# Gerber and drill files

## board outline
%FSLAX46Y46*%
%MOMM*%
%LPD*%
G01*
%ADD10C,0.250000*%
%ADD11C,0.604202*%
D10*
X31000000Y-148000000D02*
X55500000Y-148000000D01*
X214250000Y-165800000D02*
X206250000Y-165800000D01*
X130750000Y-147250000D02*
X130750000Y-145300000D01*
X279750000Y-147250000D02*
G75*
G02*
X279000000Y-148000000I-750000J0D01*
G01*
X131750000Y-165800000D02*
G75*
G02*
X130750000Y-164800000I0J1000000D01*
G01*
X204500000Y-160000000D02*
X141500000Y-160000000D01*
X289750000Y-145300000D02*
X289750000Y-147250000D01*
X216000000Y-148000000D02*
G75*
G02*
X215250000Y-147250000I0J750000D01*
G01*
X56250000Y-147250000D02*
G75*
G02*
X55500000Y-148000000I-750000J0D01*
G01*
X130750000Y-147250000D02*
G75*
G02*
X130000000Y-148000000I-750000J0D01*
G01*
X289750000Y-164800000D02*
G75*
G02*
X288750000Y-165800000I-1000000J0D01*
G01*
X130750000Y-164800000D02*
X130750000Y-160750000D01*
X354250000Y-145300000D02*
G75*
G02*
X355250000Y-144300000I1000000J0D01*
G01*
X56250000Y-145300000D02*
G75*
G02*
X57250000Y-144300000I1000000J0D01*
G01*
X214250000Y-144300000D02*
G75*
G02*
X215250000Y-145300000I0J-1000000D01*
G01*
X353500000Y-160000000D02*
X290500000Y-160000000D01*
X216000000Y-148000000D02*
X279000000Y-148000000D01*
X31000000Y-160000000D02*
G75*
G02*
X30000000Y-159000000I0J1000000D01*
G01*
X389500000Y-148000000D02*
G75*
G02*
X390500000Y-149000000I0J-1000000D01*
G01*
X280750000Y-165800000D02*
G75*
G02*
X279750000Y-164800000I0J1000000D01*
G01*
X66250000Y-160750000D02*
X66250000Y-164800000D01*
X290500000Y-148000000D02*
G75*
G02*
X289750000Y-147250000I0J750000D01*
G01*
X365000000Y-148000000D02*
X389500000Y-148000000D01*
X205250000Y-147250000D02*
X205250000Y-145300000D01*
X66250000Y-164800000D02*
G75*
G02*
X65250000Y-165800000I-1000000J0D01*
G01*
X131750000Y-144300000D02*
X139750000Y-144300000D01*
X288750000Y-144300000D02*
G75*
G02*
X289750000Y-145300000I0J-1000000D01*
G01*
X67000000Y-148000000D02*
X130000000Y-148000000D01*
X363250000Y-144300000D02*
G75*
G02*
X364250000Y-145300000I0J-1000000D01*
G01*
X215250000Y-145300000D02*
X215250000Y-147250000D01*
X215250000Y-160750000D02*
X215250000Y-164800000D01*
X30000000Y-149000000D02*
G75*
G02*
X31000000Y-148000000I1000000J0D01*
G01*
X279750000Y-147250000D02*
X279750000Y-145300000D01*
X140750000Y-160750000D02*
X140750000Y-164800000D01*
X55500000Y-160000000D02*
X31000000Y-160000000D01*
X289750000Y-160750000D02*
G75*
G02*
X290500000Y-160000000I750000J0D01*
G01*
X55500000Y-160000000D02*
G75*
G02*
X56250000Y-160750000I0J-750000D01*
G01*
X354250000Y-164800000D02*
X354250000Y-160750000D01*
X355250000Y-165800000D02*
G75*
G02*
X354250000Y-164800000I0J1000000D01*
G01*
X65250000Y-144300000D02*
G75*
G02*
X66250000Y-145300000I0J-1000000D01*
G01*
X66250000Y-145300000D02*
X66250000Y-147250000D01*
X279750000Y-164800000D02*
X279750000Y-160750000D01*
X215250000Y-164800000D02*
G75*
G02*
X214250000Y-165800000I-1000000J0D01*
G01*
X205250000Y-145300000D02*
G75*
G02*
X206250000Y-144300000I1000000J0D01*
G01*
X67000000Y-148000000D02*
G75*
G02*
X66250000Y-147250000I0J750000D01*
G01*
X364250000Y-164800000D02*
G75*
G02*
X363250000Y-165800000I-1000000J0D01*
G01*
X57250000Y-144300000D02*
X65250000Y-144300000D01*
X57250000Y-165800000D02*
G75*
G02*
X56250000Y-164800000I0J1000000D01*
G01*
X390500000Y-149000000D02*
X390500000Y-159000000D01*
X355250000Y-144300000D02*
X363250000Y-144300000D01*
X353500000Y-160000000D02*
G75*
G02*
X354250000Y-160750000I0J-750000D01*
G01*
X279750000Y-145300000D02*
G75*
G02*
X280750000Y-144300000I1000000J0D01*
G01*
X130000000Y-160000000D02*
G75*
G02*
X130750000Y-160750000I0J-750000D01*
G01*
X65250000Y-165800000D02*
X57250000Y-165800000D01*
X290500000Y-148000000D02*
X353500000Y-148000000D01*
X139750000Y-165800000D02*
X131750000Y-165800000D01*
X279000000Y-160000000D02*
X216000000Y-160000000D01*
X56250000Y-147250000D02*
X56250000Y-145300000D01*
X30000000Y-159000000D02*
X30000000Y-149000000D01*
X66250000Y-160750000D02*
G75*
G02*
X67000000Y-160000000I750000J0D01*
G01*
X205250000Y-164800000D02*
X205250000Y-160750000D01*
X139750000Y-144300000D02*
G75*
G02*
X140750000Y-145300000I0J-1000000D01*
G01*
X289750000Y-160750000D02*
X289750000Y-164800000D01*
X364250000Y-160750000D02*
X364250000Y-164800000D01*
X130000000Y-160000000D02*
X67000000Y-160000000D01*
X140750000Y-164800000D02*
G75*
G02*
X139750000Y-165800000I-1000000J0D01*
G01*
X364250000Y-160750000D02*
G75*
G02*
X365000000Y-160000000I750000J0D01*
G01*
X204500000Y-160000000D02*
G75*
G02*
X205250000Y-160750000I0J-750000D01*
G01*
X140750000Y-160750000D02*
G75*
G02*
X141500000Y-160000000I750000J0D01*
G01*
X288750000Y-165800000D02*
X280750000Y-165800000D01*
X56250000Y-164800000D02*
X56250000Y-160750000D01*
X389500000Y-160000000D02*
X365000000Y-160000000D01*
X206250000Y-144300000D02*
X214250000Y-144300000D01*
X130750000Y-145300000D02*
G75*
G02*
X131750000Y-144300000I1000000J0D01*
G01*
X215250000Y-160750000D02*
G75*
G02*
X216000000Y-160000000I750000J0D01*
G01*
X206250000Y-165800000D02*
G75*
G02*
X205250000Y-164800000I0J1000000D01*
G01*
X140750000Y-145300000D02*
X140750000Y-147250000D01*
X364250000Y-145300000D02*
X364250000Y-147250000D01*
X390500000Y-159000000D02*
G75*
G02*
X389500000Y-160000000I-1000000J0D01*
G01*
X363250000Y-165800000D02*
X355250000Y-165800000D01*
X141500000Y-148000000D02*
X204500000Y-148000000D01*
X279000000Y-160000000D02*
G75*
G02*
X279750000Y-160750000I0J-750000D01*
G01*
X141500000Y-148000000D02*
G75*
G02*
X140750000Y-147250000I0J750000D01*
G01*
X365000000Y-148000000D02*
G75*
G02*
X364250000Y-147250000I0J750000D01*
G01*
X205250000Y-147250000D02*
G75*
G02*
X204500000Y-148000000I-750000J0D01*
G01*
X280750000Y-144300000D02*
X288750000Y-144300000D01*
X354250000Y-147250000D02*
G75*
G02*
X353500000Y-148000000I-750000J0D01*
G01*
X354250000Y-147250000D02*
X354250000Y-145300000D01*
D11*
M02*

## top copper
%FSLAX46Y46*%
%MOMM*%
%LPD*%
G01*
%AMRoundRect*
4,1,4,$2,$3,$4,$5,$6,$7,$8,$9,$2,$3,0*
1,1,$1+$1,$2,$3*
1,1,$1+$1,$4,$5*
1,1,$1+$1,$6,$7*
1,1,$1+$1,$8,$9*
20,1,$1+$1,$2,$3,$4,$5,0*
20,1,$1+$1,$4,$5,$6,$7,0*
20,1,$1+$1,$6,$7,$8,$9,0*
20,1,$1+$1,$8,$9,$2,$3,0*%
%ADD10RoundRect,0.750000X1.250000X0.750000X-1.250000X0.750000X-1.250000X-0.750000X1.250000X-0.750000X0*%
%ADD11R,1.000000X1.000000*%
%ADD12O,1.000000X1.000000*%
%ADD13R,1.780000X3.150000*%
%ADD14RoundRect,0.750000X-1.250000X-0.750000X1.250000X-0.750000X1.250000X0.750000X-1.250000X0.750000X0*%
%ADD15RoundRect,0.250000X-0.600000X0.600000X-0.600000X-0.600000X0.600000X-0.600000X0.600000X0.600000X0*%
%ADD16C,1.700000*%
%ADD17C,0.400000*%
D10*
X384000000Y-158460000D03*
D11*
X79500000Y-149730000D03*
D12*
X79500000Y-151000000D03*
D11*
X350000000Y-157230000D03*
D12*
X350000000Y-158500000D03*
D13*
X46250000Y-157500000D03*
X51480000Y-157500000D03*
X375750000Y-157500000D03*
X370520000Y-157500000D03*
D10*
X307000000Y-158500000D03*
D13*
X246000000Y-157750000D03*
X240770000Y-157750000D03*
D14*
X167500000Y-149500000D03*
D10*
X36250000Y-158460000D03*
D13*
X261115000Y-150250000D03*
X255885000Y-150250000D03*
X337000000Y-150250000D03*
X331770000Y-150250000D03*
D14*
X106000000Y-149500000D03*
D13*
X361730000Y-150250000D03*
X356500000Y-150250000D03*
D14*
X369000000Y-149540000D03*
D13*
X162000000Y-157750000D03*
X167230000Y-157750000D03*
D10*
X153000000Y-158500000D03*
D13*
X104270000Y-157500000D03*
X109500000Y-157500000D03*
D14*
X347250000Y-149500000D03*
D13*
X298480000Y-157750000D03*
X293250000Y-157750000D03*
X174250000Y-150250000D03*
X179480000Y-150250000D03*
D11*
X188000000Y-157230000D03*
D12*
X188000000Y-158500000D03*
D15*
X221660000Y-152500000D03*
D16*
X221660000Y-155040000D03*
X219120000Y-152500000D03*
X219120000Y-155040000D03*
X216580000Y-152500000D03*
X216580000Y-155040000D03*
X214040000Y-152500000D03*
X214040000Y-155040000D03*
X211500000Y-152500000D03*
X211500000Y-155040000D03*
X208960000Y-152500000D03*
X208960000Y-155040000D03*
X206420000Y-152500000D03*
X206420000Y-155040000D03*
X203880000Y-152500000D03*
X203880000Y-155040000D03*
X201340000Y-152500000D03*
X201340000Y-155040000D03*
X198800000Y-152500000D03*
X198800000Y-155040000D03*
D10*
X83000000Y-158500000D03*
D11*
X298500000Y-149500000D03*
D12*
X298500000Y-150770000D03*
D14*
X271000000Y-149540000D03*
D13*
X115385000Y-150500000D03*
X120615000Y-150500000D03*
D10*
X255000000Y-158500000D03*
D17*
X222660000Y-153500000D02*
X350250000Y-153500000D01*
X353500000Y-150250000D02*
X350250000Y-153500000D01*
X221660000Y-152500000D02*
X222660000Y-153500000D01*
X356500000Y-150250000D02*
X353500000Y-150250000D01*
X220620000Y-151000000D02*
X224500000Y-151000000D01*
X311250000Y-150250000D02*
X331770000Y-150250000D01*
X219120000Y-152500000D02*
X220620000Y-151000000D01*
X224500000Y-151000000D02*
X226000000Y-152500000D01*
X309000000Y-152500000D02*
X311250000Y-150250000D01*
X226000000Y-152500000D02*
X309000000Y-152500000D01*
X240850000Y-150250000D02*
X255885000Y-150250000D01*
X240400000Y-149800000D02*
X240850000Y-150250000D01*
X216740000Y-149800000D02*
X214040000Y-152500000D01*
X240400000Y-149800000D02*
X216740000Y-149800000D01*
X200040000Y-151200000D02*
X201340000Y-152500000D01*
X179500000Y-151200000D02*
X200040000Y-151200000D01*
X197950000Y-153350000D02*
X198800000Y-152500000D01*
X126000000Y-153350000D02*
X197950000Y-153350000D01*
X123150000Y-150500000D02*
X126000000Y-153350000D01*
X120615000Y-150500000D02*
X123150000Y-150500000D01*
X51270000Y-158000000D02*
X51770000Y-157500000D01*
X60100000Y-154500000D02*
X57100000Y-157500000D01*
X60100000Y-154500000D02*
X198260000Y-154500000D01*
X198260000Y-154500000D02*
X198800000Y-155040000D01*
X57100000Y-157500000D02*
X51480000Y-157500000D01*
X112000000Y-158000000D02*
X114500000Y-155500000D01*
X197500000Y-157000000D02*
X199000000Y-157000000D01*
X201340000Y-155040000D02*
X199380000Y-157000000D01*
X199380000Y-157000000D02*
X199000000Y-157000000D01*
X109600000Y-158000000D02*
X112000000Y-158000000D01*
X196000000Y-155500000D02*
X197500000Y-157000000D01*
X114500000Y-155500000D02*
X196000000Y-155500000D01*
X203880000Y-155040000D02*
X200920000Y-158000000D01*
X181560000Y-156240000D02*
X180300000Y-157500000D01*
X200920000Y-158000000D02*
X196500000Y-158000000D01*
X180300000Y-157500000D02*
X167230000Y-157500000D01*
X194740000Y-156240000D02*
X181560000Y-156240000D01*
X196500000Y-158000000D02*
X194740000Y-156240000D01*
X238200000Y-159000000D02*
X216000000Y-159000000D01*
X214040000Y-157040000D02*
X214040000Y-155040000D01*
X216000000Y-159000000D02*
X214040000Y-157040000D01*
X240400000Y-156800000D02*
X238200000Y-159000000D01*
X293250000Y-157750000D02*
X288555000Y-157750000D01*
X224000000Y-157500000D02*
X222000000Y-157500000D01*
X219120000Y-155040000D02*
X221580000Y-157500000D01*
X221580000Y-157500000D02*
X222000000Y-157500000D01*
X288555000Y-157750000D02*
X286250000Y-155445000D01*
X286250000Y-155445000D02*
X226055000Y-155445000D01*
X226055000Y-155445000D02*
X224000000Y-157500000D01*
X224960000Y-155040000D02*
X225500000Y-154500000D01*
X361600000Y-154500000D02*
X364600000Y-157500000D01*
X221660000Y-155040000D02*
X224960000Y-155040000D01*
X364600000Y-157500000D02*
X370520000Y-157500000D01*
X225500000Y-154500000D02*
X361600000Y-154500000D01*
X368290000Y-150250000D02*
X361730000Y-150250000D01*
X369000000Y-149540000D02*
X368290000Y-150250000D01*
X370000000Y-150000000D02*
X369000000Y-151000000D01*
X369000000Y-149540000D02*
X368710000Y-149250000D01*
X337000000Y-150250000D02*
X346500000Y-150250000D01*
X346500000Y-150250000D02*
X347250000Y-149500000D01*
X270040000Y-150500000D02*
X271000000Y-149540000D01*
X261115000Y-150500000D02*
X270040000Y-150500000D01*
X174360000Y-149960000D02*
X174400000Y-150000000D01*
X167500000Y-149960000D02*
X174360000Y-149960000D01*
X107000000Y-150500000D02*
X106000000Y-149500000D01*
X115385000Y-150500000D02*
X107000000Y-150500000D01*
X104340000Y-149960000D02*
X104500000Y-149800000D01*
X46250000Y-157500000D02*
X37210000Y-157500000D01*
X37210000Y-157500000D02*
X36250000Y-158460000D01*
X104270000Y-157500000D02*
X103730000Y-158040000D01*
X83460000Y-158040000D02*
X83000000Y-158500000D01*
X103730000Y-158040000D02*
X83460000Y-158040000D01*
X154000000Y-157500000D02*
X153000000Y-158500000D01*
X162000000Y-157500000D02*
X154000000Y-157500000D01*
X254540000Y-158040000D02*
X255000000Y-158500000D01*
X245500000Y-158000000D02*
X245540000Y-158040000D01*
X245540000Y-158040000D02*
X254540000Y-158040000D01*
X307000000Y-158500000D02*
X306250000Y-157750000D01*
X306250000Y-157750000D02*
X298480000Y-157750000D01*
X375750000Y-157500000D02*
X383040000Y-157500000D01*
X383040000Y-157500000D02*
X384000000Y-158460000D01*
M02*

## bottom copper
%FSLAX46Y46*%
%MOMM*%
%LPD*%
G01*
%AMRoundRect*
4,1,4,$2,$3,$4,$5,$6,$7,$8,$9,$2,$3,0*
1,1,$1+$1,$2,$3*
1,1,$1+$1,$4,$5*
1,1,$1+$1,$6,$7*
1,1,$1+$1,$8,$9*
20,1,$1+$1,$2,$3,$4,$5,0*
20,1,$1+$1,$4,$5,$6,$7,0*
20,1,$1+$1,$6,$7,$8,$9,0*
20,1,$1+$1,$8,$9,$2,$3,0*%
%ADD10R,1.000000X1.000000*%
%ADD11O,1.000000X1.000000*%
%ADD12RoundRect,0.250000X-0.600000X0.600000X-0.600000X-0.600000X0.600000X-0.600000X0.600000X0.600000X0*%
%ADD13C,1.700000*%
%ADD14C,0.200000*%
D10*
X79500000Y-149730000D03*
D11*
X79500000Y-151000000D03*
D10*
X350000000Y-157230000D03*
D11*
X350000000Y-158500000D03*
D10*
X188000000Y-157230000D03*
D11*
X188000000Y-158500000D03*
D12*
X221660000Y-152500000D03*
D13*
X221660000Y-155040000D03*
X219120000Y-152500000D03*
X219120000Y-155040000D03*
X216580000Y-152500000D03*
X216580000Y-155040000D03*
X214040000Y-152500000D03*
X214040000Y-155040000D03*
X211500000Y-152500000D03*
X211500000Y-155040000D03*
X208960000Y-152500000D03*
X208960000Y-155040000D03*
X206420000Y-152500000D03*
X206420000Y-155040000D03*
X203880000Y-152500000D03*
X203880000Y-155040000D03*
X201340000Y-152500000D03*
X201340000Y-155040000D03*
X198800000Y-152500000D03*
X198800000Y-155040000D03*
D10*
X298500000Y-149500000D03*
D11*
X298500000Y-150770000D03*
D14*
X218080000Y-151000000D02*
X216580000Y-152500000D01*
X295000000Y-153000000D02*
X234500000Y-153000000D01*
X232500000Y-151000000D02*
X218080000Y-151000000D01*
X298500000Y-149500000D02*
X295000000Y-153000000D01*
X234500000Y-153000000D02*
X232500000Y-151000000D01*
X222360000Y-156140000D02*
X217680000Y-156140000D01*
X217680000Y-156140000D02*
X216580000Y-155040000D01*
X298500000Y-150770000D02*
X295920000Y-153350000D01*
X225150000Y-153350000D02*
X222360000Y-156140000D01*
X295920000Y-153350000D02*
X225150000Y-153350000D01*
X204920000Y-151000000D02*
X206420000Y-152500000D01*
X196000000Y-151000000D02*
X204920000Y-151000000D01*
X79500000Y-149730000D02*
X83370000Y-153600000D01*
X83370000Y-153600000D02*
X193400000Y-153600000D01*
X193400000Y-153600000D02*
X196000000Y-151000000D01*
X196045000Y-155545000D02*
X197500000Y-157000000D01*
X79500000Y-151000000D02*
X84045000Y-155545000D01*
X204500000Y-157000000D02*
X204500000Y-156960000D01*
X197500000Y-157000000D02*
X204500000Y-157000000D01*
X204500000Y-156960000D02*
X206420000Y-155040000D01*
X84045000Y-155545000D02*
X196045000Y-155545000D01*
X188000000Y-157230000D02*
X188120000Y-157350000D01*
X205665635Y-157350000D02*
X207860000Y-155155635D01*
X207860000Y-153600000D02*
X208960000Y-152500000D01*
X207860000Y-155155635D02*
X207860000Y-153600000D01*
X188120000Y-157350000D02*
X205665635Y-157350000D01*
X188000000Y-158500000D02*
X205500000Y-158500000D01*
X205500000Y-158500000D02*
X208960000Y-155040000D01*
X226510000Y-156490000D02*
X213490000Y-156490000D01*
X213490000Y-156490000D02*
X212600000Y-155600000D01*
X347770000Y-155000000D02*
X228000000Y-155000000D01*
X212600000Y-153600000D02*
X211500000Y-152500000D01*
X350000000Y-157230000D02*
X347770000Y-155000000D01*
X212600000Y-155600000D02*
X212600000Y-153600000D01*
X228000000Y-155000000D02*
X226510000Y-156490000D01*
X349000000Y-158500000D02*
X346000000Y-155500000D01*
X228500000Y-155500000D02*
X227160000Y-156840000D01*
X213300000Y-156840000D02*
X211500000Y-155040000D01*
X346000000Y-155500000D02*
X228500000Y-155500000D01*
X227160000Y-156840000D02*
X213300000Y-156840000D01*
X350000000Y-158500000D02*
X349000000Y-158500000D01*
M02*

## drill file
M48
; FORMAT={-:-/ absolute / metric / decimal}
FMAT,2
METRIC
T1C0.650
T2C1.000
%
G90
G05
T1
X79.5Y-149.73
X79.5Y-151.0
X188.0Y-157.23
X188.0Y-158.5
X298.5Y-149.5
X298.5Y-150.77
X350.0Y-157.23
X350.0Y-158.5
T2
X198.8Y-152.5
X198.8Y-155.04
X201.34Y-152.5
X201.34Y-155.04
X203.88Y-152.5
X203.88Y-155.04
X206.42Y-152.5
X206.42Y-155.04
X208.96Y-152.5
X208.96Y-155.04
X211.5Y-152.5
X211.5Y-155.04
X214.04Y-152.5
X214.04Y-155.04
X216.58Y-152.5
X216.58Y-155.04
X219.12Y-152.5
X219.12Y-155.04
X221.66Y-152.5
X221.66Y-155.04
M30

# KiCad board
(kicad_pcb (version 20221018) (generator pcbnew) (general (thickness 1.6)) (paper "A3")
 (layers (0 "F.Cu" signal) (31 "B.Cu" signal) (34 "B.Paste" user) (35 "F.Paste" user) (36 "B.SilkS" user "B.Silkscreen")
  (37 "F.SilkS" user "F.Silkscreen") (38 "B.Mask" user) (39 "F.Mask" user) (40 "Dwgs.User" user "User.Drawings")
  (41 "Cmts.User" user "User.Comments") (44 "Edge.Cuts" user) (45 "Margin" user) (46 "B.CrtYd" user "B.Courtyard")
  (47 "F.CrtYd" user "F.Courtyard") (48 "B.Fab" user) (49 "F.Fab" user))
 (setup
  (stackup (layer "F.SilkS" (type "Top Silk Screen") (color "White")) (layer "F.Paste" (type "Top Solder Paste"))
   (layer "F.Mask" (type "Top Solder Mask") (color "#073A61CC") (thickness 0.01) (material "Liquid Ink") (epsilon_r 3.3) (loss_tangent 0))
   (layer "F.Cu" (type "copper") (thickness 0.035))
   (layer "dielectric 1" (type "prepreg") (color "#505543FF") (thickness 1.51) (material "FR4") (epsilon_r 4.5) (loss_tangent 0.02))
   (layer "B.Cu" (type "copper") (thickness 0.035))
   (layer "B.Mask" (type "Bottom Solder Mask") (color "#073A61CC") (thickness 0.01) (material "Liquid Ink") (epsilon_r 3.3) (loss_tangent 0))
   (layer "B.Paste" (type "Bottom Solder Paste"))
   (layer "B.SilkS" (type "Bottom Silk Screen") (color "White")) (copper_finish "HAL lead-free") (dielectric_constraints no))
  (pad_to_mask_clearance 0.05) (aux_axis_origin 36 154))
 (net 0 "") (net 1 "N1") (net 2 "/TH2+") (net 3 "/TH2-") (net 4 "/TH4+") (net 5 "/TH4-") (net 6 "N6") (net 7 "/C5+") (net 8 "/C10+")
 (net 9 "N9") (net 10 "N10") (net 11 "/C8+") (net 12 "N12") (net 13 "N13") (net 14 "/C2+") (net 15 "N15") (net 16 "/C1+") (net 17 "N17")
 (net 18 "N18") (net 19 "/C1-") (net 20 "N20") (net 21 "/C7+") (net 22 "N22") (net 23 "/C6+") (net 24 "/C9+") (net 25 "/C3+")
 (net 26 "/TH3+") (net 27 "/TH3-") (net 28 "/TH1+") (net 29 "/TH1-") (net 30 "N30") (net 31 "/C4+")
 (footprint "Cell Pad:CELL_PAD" (layer "F.Cu") (at 384 158.46 180)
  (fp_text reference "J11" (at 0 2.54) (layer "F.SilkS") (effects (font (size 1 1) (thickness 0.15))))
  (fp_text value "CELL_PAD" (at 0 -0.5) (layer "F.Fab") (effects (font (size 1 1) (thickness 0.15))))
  (pad "1" smd roundrect (at 0 0 180) (size 4 3) (layers "F.Cu" "F.Paste" "F.Mask") (roundrect_rratio 0.25) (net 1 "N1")))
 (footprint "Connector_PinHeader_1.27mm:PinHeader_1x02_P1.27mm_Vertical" (layer "F.Cu") (at 79.5 149.73)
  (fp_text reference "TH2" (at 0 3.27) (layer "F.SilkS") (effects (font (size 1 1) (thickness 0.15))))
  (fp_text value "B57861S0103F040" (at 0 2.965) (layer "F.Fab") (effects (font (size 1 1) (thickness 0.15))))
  (pad "1" thru_hole rect (at 0 0) (size 1 1) (drill 0.65) (layers "*.Cu" "*.Mask") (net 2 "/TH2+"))
  (pad "2" thru_hole oval (at 0 1.27) (size 1 1) (drill 0.65) (layers "*.Cu" "*.Mask") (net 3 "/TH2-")))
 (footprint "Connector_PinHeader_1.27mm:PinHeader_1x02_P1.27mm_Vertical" (layer "F.Cu") (at 350 157.23)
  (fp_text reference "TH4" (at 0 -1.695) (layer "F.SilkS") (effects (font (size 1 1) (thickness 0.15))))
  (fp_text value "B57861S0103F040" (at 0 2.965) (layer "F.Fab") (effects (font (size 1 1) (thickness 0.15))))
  (pad "1" thru_hole rect (at 0 0) (size 1 1) (drill 0.65) (layers "*.Cu" "*.Mask") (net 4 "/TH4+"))
  (pad "2" thru_hole oval (at 0 1.27) (size 1 1) (drill 0.65) (layers "*.Cu" "*.Mask") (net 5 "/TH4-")))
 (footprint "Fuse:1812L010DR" (layer "F.Cu") (at 48.865 157.5)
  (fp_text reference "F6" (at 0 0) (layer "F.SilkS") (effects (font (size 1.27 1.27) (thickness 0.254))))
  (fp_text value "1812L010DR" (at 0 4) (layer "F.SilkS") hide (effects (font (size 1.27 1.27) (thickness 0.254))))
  (pad "1" smd rect (at -2.615 0) (size 1.78 3.15) (layers "F.Cu" "F.Paste" "F.Mask") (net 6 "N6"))
  (pad "2" smd rect (at 2.615 0) (size 1.78 3.15) (layers "F.Cu" "F.Paste" "F.Mask") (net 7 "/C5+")))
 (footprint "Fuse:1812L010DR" (layer "F.Cu") (at 373.135 157.5 180)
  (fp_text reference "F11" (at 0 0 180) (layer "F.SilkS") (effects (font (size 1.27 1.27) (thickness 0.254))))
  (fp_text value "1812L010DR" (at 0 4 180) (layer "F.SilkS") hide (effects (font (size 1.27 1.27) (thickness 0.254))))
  (pad "1" smd rect (at -2.615 0 180) (size 1.78 3.15) (layers "F.Cu" "F.Paste" "F.Mask") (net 1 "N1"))
  (pad "2" smd rect (at 2.615 0 180) (size 1.78 3.15) (layers "F.Cu" "F.Paste" "F.Mask") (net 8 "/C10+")))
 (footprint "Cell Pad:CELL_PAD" (layer "F.Cu") (at 307 158.5 180)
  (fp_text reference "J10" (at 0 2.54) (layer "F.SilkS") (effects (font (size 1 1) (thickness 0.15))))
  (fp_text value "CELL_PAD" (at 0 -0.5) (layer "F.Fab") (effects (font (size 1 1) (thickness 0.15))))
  (pad "1" smd roundrect (at 0 0 180) (size 4 3) (layers "F.Cu" "F.Paste" "F.Mask") (roundrect_rratio 0.25) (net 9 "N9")))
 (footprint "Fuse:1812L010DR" (layer "F.Cu") (at 243.385 157.75 180)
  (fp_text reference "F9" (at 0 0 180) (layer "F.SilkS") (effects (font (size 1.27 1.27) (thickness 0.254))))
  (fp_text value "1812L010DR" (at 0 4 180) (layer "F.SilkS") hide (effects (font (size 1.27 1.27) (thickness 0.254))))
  (pad "1" smd rect (at -2.615 0 180) (size 1.78 3.15) (layers "F.Cu" "F.Paste" "F.Mask") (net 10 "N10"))
  (pad "2" smd rect (at 2.615 0 180) (size 1.78 3.15) (layers "F.Cu" "F.Paste" "F.Mask") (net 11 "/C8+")))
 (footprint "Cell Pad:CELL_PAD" (layer "F.Cu") (at 167.5 149.5)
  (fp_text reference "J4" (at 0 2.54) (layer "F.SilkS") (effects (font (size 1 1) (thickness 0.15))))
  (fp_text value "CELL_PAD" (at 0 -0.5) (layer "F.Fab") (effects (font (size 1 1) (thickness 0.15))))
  (pad "1" smd roundrect (at 0 0) (size 4 3) (layers "F.Cu" "F.Paste" "F.Mask") (roundrect_rratio 0.25) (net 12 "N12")))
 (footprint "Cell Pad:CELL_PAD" (layer "F.Cu") (at 36.25 158.46 180)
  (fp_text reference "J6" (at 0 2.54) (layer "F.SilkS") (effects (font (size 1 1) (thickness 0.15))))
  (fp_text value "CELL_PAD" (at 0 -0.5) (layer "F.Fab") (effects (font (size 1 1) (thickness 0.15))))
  (pad "1" smd roundrect (at 0 0 180) (size 4 3) (layers "F.Cu" "F.Paste" "F.Mask") (roundrect_rratio 0.25) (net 6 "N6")))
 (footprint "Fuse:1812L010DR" (layer "F.Cu") (at 258.5 150.25 180)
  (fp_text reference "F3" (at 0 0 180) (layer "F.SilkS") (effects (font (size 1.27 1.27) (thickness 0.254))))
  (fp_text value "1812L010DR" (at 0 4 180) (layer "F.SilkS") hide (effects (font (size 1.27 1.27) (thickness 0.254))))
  (pad "1" smd rect (at -2.615 0 180) (size 1.78 3.15) (layers "F.Cu" "F.Paste" "F.Mask") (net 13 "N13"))
  (pad "2" smd rect (at 2.615 0 180) (size 1.78 3.15) (layers "F.Cu" "F.Paste" "F.Mask") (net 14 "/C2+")))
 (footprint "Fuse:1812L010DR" (layer "F.Cu") (at 334.385 150.25 180)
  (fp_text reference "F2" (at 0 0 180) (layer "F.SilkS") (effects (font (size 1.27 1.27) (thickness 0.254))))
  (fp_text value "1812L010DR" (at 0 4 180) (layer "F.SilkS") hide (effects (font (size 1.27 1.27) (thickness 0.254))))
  (pad "1" smd rect (at -2.615 0 180) (size 1.78 3.15) (layers "F.Cu" "F.Paste" "F.Mask") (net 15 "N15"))
  (pad "2" smd rect (at 2.615 0 180) (size 1.78 3.15) (layers "F.Cu" "F.Paste" "F.Mask") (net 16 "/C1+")))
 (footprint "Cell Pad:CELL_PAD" (layer "F.Cu") (at 106 149.5)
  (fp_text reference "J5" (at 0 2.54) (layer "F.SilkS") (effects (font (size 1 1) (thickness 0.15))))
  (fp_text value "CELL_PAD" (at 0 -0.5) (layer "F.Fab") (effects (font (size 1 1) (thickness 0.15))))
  (pad "1" smd roundrect (at 0 0) (size 4 3) (layers "F.Cu" "F.Paste" "F.Mask") (roundrect_rratio 0.25) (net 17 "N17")))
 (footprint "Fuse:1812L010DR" (layer "F.Cu") (at 359.115 150.25 180)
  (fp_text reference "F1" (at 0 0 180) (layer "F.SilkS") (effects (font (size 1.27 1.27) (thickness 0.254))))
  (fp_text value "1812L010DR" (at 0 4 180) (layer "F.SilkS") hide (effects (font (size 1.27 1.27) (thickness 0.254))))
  (pad "1" smd rect (at -2.615 0 180) (size 1.78 3.15) (layers "F.Cu" "F.Paste" "F.Mask") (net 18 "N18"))
  (pad "2" smd rect (at 2.615 0 180) (size 1.78 3.15) (layers "F.Cu" "F.Paste" "F.Mask") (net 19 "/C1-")))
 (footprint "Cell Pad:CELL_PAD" (layer "F.Cu") (at 369 149.54)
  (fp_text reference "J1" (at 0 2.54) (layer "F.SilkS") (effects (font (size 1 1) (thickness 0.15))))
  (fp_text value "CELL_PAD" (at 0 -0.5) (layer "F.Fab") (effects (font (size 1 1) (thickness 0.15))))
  (pad "1" smd roundrect (at 0 0) (size 4 3) (layers "F.Cu" "F.Paste" "F.Mask") (roundrect_rratio 0.25) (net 18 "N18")))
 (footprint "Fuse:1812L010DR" (layer "F.Cu") (at 164.615 157.75)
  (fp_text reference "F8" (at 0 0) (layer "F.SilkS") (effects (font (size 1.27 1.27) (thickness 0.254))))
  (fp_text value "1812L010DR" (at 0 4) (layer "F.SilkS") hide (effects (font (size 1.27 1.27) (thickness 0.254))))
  (pad "1" smd rect (at -2.615 0) (size 1.78 3.15) (layers "F.Cu" "F.Paste" "F.Mask") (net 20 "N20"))
  (pad "2" smd rect (at 2.615 0) (size 1.78 3.15) (layers "F.Cu" "F.Paste" "F.Mask") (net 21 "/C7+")))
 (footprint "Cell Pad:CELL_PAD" (layer "F.Cu") (at 153 158.5 180)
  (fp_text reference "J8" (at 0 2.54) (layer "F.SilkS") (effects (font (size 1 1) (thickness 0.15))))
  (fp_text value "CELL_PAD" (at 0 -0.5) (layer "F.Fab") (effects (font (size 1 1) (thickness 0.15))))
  (pad "1" smd roundrect (at 0 0 180) (size 4 3) (layers "F.Cu" "F.Paste" "F.Mask") (roundrect_rratio 0.25) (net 20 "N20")))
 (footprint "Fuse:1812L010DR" (layer "F.Cu") (at 106.885 157.5)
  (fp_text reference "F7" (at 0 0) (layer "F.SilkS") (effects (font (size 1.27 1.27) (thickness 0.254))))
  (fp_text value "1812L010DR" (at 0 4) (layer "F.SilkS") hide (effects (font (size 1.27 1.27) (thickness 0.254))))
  (pad "1" smd rect (at -2.615 0) (size 1.78 3.15) (layers "F.Cu" "F.Paste" "F.Mask") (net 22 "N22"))
  (pad "2" smd rect (at 2.615 0) (size 1.78 3.15) (layers "F.Cu" "F.Paste" "F.Mask") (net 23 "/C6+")))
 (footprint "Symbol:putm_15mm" (layer "F.Cu") (at 136 154)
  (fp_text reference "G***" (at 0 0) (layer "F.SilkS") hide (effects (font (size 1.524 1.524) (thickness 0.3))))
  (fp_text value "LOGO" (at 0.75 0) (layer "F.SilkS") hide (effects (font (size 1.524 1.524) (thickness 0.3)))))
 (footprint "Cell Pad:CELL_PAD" (layer "F.Cu") (at 347.25 149.5)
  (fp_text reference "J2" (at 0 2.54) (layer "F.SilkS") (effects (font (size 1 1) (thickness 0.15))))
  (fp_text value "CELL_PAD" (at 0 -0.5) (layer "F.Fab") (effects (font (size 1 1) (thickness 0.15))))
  (pad "1" smd roundrect (at 0 0) (size 4 3) (layers "F.Cu" "F.Paste" "F.Mask") (roundrect_rratio 0.25) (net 15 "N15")))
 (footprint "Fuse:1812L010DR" (layer "F.Cu") (at 295.865 157.75 180)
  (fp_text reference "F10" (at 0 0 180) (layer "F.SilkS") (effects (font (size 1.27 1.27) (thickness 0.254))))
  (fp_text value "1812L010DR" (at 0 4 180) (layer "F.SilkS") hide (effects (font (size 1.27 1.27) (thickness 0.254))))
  (pad "1" smd rect (at -2.615 0 180) (size 1.78 3.15) (layers "F.Cu" "F.Paste" "F.Mask") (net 9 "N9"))
  (pad "2" smd rect (at 2.615 0 180) (size 1.78 3.15) (layers "F.Cu" "F.Paste" "F.Mask") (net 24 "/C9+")))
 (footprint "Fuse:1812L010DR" (layer "F.Cu") (at 176.865 150.25)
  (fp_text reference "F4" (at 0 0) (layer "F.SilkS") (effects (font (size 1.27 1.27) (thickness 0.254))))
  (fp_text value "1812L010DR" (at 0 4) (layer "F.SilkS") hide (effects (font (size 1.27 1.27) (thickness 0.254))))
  (pad "1" smd rect (at -2.615 0) (size 1.78 3.15) (layers "F.Cu" "F.Paste" "F.Mask") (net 12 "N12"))
  (pad "2" smd rect (at 2.615 0) (size 1.78 3.15) (layers "F.Cu" "F.Paste" "F.Mask") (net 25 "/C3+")))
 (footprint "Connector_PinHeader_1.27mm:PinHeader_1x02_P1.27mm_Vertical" (layer "F.Cu") (at 188 157.23)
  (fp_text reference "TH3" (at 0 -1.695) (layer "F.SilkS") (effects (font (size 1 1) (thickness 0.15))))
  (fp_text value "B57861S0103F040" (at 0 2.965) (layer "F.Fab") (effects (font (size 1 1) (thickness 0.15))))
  (pad "1" thru_hole rect (at 0 0) (size 1 1) (drill 0.65) (layers "*.Cu" "*.Mask") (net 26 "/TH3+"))
  (pad "2" thru_hole oval (at 0 1.27) (size 1 1) (drill 0.65) (layers "*.Cu" "*.Mask") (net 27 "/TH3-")))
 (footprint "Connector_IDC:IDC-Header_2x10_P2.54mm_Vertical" (layer "F.Cu") (at 221.66 152.5 -90)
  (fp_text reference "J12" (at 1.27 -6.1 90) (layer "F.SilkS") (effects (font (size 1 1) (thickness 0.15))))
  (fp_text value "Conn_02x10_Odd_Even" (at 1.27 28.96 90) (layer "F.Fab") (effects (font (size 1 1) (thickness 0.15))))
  (pad "1" thru_hole roundrect (at 0 0 270) (size 1.7 1.7) (drill 1) (layers "*.Cu" "*.Mask") (roundrect_rratio 0.147059) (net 19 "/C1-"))
  (pad "2" thru_hole circle (at 2.54 0 270) (size 1.7 1.7) (drill 1) (layers "*.Cu" "*.Mask") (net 8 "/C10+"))
  (pad "3" thru_hole circle (at 0 2.54 270) (size 1.7 1.7) (drill 1) (layers "*.Cu" "*.Mask") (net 16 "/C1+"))
  (pad "4" thru_hole circle (at 2.54 2.54 270) (size 1.7 1.7) (drill 1) (layers "*.Cu" "*.Mask") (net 24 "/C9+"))
  (pad "5" thru_hole circle (at 0 5.08 270) (size 1.7 1.7) (drill 1) (layers "*.Cu" "*.Mask") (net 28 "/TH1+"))
  (pad "6" thru_hole circle (at 2.54 5.08 270) (size 1.7 1.7) (drill 1) (layers "*.Cu" "*.Mask") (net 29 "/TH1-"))
  (pad "7" thru_hole circle (at 0 7.62 270) (size 1.7 1.7) (drill 1) (layers "*.Cu" "*.Mask") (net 14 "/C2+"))
  (pad "8" thru_hole circle (at 2.54 7.62 270) (size 1.7 1.7) (drill 1) (layers "*.Cu" "*.Mask") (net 11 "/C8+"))
  (pad "9" thru_hole circle (at 0 10.16 270) (size 1.7 1.7) (drill 1) (layers "*.Cu" "*.Mask") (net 4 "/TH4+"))
  (pad "10" thru_hole circle (at 2.54 10.16 270) (size 1.7 1.7) (drill 1) (layers "*.Cu" "*.Mask") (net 5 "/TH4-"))
  (pad "11" thru_hole circle (at 0 12.7 270) (size 1.7 1.7) (drill 1) (layers "*.Cu" "*.Mask") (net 26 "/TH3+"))
  (pad "12" thru_hole circle (at 2.54 12.7 270) (size 1.7 1.7) (drill 1) (layers "*.Cu" "*.Mask") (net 27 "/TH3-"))
  (pad "13" thru_hole circle (at 0 15.24 270) (size 1.7 1.7) (drill 1) (layers "*.Cu" "*.Mask") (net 2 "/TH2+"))
  (pad "14" thru_hole circle (at 2.54 15.24 270) (size 1.7 1.7) (drill 1) (layers "*.Cu" "*.Mask") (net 3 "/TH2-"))
  (pad "15" thru_hole circle (at 0 17.78 270) (size 1.7 1.7) (drill 1) (layers "*.Cu" "*.Mask") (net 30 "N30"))
  (pad "16" thru_hole circle (at 2.54 17.78 270) (size 1.7 1.7) (drill 1) (layers "*.Cu" "*.Mask") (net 21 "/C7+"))
  (pad "17" thru_hole circle (at 0 20.32 270) (size 1.7 1.7) (drill 1) (layers "*.Cu" "*.Mask") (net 25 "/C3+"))
  (pad "18" thru_hole circle (at 2.54 20.32 270) (size 1.7 1.7) (drill 1) (layers "*.Cu" "*.Mask") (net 23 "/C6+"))
  (pad "19" thru_hole circle (at 0 22.86 270) (size 1.7 1.7) (drill 1) (layers "*.Cu" "*.Mask") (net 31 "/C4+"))
  (pad "20" thru_hole circle (at 2.54 22.86 270) (size 1.7 1.7) (drill 1) (layers "*.Cu" "*.Mask") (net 7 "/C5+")))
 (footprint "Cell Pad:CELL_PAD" (layer "F.Cu") (at 83 158.5 180)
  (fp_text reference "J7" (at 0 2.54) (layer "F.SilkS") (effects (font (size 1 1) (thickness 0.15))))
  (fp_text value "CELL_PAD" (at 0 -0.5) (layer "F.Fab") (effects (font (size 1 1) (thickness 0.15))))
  (pad "1" smd roundrect (at 0 0 180) (size 4 3) (layers "F.Cu" "F.Paste" "F.Mask") (roundrect_rratio 0.25) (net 22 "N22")))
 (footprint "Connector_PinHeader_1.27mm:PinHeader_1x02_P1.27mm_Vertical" (layer "F.Cu") (at 298.5 149.5)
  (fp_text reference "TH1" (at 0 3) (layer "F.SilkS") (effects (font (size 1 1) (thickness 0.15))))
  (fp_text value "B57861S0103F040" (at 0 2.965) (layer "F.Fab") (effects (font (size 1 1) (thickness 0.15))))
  (pad "1" thru_hole rect (at 0 0) (size 1 1) (drill 0.65) (layers "*.Cu" "*.Mask") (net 28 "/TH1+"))
  (pad "2" thru_hole oval (at 0 1.27) (size 1 1) (drill 0.65) (layers "*.Cu" "*.Mask") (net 29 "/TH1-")))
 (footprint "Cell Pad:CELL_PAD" (layer "F.Cu") (at 271 149.54)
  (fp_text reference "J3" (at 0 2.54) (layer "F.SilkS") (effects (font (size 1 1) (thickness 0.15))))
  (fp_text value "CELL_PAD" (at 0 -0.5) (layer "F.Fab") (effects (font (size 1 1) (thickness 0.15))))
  (pad "1" smd roundrect (at 0 0) (size 4 3) (layers "F.Cu" "F.Paste" "F.Mask") (roundrect_rratio 0.25) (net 13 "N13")))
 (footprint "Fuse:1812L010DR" (layer "F.Cu") (at 118 150.5)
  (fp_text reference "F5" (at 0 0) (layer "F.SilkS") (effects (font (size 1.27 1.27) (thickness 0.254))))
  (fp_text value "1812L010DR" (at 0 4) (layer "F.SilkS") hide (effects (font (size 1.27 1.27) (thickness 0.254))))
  (pad "1" smd rect (at -2.615 0) (size 1.78 3.15) (layers "F.Cu" "F.Paste" "F.Mask") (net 17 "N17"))
  (pad "2" smd rect (at 2.615 0) (size 1.78 3.15) (layers "F.Cu" "F.Paste" "F.Mask") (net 31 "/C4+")))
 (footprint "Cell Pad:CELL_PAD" (layer "F.Cu") (at 255 158.5 180)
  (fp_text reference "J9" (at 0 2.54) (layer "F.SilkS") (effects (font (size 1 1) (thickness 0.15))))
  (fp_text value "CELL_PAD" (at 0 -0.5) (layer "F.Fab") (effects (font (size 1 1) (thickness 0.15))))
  (pad "1" smd roundrect (at 0 0 180) (size 4 3) (layers "F.Cu" "F.Paste" "F.Mask") (roundrect_rratio 0.25) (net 10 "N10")))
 (gr_line (start 31 148) (end 55.5 148) (stroke (width 0.25) (type solid)) (layer "Edge.Cuts"))
 (gr_line (start 214.25 165.8) (end 206.25 165.8) (stroke (width 0.25) (type solid)) (layer "Edge.Cuts"))
 (gr_line (start 130.75 147.25) (end 130.75 145.3) (stroke (width 0.25) (type solid)) (layer "Edge.Cuts"))
 (gr_arc (start 279.75 147.25) (mid 279.53033 147.78033) (end 279 148) (stroke (width 0.25) (type solid)) (layer "Edge.Cuts"))
 (gr_arc (start 131.75 165.8) (mid 131.042893 165.507107) (end 130.75 164.8) (stroke (width 0.25) (type solid)) (layer "Edge.Cuts"))
 (gr_line (start 204.5 160) (end 141.5 160) (stroke (width 0.25) (type solid)) (layer "Edge.Cuts"))
 (gr_line (start 289.75 145.3) (end 289.75 147.25) (stroke (width 0.25) (type solid)) (layer "Edge.Cuts"))
 (gr_arc (start 216 148) (mid 215.46967 147.78033) (end 215.25 147.25) (stroke (width 0.25) (type solid)) (layer "Edge.Cuts"))
 (gr_arc (start 56.25 147.25) (mid 56.03033 147.78033) (end 55.5 148) (stroke (width 0.25) (type solid)) (layer "Edge.Cuts"))
 (gr_arc (start 130.75 147.25) (mid 130.53033 147.78033) (end 130 148) (stroke (width 0.25) (type solid)) (layer "Edge.Cuts"))
 (gr_arc (start 289.75 164.8) (mid 289.457107 165.507107) (end 288.75 165.8) (stroke (width 0.25) (type solid)) (layer "Edge.Cuts"))
 (gr_line (start 130.75 164.8) (end 130.75 160.75) (stroke (width 0.25) (type solid)) (layer "Edge.Cuts"))
 (gr_arc (start 354.25 145.3) (mid 354.542893 144.592893) (end 355.25 144.3) (stroke (width 0.25) (type solid)) (layer "Edge.Cuts"))
 (gr_arc (start 56.25 145.3) (mid 56.542893 144.592893) (end 57.25 144.3) (stroke (width 0.25) (type solid)) (layer "Edge.Cuts"))
 (gr_arc (start 214.25 144.3) (mid 214.957107 144.592893) (end 215.25 145.3) (stroke (width 0.25) (type solid)) (layer "Edge.Cuts"))
 (gr_line (start 353.5 160) (end 290.5 160) (stroke (width 0.25) (type solid)) (layer "Edge.Cuts"))
 (gr_line (start 216 148) (end 279 148) (stroke (width 0.25) (type solid)) (layer "Edge.Cuts"))
 (gr_arc (start 31 160) (mid 30.292893 159.707107) (end 30 159) (stroke (width 0.25) (type solid)) (layer "Edge.Cuts"))
 (gr_arc (start 389.5 148) (mid 390.207107 148.292893) (end 390.5 149) (stroke (width 0.25) (type solid)) (layer "Edge.Cuts"))
 (gr_arc (start 280.75 165.8) (mid 280.042893 165.507107) (end 279.75 164.8) (stroke (width 0.25) (type solid)) (layer "Edge.Cuts"))
 (gr_line (start 66.25 160.75) (end 66.25 164.8) (stroke (width 0.25) (type solid)) (layer "Edge.Cuts"))
 (gr_arc (start 290.5 148) (mid 289.96967 147.78033) (end 289.75 147.25) (stroke (width 0.25) (type solid)) (layer "Edge.Cuts"))
 (gr_line (start 365 148) (end 389.5 148) (stroke (width 0.25) (type solid)) (layer "Edge.Cuts"))
 (gr_line (start 205.25 147.25) (end 205.25 145.3) (stroke (width 0.25) (type solid)) (layer "Edge.Cuts"))
 (gr_arc (start 66.25 164.8) (mid 65.957107 165.507107) (end 65.25 165.8) (stroke (width 0.25) (type solid)) (layer "Edge.Cuts"))
 (gr_line (start 131.75 144.3) (end 139.75 144.3) (stroke (width 0.25) (type solid)) (layer "Edge.Cuts"))
 (gr_arc (start 288.75 144.3) (mid 289.457107 144.592893) (end 289.75 145.3) (stroke (width 0.25) (type solid)) (layer "Edge.Cuts"))
 (gr_line (start 67 148) (end 130 148) (stroke (width 0.25) (type solid)) (layer "Edge.Cuts"))
 (gr_arc (start 363.25 144.3) (mid 363.957107 144.592893) (end 364.25 145.3) (stroke (width 0.25) (type solid)) (layer "Edge.Cuts"))
 (gr_line (start 215.25 145.3) (end 215.25 147.25) (stroke (width 0.25) (type solid)) (layer "Edge.Cuts"))
 (gr_line (start 215.25 160.75) (end 215.25 164.8) (stroke (width 0.25) (type solid)) (layer "Edge.Cuts"))
 (gr_arc (start 30 149) (mid 30.292893 148.292893) (end 31 148) (stroke (width 0.25) (type solid)) (layer "Edge.Cuts"))
 (gr_line (start 279.75 147.25) (end 279.75 145.3) (stroke (width 0.25) (type solid)) (layer "Edge.Cuts"))
 (gr_line (start 140.75 160.75) (end 140.75 164.8) (stroke (width 0.25) (type solid)) (layer "Edge.Cuts"))
 (gr_line (start 55.5 160) (end 31 160) (stroke (width 0.25) (type solid)) (layer "Edge.Cuts"))
 (gr_arc (start 289.75 160.75) (mid 289.96967 160.21967) (end 290.5 160) (stroke (width 0.25) (type solid)) (layer "Edge.Cuts"))
 (gr_arc (start 55.5 160) (mid 56.03033 160.21967) (end 56.25 160.75) (stroke (width 0.25) (type solid)) (layer "Edge.Cuts"))
 (gr_line (start 354.25 164.8) (end 354.25 160.75) (stroke (width 0.25) (type solid)) (layer "Edge.Cuts"))
 (gr_arc (start 355.25 165.8) (mid 354.542893 165.507107) (end 354.25 164.8) (stroke (width 0.25) (type solid)) (layer "Edge.Cuts"))
 (gr_arc (start 65.25 144.3) (mid 65.957107 144.592893) (end 66.25 145.3) (stroke (width 0.25) (type solid)) (layer "Edge.Cuts"))
 (gr_line (start 66.25 145.3) (end 66.25 147.25) (stroke (width 0.25) (type solid)) (layer "Edge.Cuts"))
 (gr_line (start 279.75 164.8) (end 279.75 160.75) (stroke (width 0.25) (type solid)) (layer "Edge.Cuts"))
 (gr_arc (start 215.25 164.8) (mid 214.957107 165.507107) (end 214.25 165.8) (stroke (width 0.25) (type solid)) (layer "Edge.Cuts"))
 (gr_arc (start 205.25 145.3) (mid 205.542893 144.592893) (end 206.25 144.3) (stroke (width 0.25) (type solid)) (layer "Edge.Cuts"))
 (gr_arc (start 67 148) (mid 66.46967 147.78033) (end 66.25 147.25) (stroke (width 0.25) (type solid)) (layer "Edge.Cuts"))
 (gr_arc (start 364.25 164.8) (mid 363.957107 165.507107) (end 363.25 165.8) (stroke (width 0.25) (type solid)) (layer "Edge.Cuts"))
 (gr_line (start 57.25 144.3) (end 65.25 144.3) (stroke (width 0.25) (type solid)) (layer "Edge.Cuts"))
 (gr_arc (start 57.25 165.8) (mid 56.542893 165.507107) (end 56.25 164.8) (stroke (width 0.25) (type solid)) (layer "Edge.Cuts"))
 (gr_line (start 390.5 149) (end 390.5 159) (stroke (width 0.25) (type solid)) (layer "Edge.Cuts"))
 (gr_line (start 355.25 144.3) (end 363.25 144.3) (stroke (width 0.25) (type solid)) (layer "Edge.Cuts"))
 (gr_arc (start 353.5 160) (mid 354.03033 160.21967) (end 354.25 160.75) (stroke (width 0.25) (type solid)) (layer "Edge.Cuts"))
 (gr_arc (start 279.75 145.3) (mid 280.042893 144.592893) (end 280.75 144.3) (stroke (width 0.25) (type solid)) (layer "Edge.Cuts"))
 (gr_arc (start 130 160) (mid 130.53033 160.21967) (end 130.75 160.75) (stroke (width 0.25) (type solid)) (layer "Edge.Cuts"))
 (gr_line (start 65.25 165.8) (end 57.25 165.8) (stroke (width 0.25) (type solid)) (layer "Edge.Cuts"))
 (gr_line (start 290.5 148) (end 353.5 148) (stroke (width 0.25) (type solid)) (layer "Edge.Cuts"))
 (gr_line (start 139.75 165.8) (end 131.75 165.8) (stroke (width 0.25) (type solid)) (layer "Edge.Cuts"))
 (gr_line (start 279 160) (end 216 160) (stroke (width 0.25) (type solid)) (layer "Edge.Cuts"))
 (gr_line (start 56.25 147.25) (end 56.25 145.3) (stroke (width 0.25) (type solid)) (layer "Edge.Cuts"))
 (gr_line (start 30 159) (end 30 149) (stroke (width 0.25) (type solid)) (layer "Edge.Cuts"))
 (gr_arc (start 66.25 160.75) (mid 66.46967 160.21967) (end 67 160) (stroke (width 0.25) (type solid)) (layer "Edge.Cuts"))
 (gr_line (start 205.25 164.8) (end 205.25 160.75) (stroke (width 0.25) (type solid)) (layer "Edge.Cuts"))
 (gr_arc (start 139.75 144.3) (mid 140.457107 144.592893) (end 140.75 145.3) (stroke (width 0.25) (type solid)) (layer "Edge.Cuts"))
 (gr_line (start 289.75 160.75) (end 289.75 164.8) (stroke (width 0.25) (type solid)) (layer "Edge.Cuts"))
 (gr_line (start 364.25 160.75) (end 364.25 164.8) (stroke (width 0.25) (type solid)) (layer "Edge.Cuts"))
 (gr_line (start 130 160) (end 67 160) (stroke (width 0.25) (type solid)) (layer "Edge.Cuts"))
 (gr_arc (start 140.75 164.8) (mid 140.457107 165.507107) (end 139.75 165.8) (stroke (width 0.25) (type solid)) (layer "Edge.Cuts"))
 (gr_arc (start 364.25 160.75) (mid 364.46967 160.21967) (end 365 160) (stroke (width 0.25) (type solid)) (layer "Edge.Cuts"))
 (gr_arc (start 204.5 160) (mid 205.03033 160.21967) (end 205.25 160.75) (stroke (width 0.25) (type solid)) (layer "Edge.Cuts"))
 (gr_arc (start 140.75 160.75) (mid 140.96967 160.21967) (end 141.5 160) (stroke (width 0.25) (type solid)) (layer "Edge.Cuts"))
 (gr_line (start 288.75 165.8) (end 280.75 165.8) (stroke (width 0.25) (type solid)) (layer "Edge.Cuts"))
 (gr_line (start 56.25 164.8) (end 56.25 160.75) (stroke (width 0.25) (type solid)) (layer "Edge.Cuts"))
 (gr_line (start 389.5 160) (end 365 160) (stroke (width 0.25) (type solid)) (layer "Edge.Cuts"))
 (gr_line (start 206.25 144.3) (end 214.25 144.3) (stroke (width 0.25) (type solid)) (layer "Edge.Cuts"))
 (gr_arc (start 130.75 145.3) (mid 131.042893 144.592893) (end 131.75 144.3) (stroke (width 0.25) (type solid)) (layer "Edge.Cuts"))
 (gr_arc (start 215.25 160.75) (mid 215.46967 160.21967) (end 216 160) (stroke (width 0.25) (type solid)) (layer "Edge.Cuts"))
 (gr_arc (start 206.25 165.8) (mid 205.542893 165.507107) (end 205.25 164.8) (stroke (width 0.25) (type solid)) (layer "Edge.Cuts"))
 (gr_line (start 140.75 145.3) (end 140.75 147.25) (stroke (width 0.25) (type solid)) (layer "Edge.Cuts"))
 (gr_line (start 364.25 145.3) (end 364.25 147.25) (stroke (width 0.25) (type solid)) (layer "Edge.Cuts"))
 (gr_arc (start 390.5 159) (mid 390.207107 159.707107) (end 389.5 160) (stroke (width 0.25) (type solid)) (layer "Edge.Cuts"))
 (gr_line (start 363.25 165.8) (end 355.25 165.8) (stroke (width 0.25) (type solid)) (layer "Edge.Cuts"))
 (gr_line (start 141.5 148) (end 204.5 148) (stroke (width 0.25) (type solid)) (layer "Edge.Cuts"))
 (gr_arc (start 279 160) (mid 279.53033 160.21967) (end 279.75 160.75) (stroke (width 0.25) (type solid)) (layer "Edge.Cuts"))
 (gr_arc (start 141.5 148) (mid 140.96967 147.78033) (end 140.75 147.25) (stroke (width 0.25) (type solid)) (layer "Edge.Cuts"))
 (gr_arc (start 365 148) (mid 364.46967 147.78033) (end 364.25 147.25) (stroke (width 0.25) (type solid)) (layer "Edge.Cuts"))
 (gr_arc (start 205.25 147.25) (mid 205.03033 147.78033) (end 204.5 148) (stroke (width 0.25) (type solid)) (layer "Edge.Cuts"))
 (gr_line (start 280.75 144.3) (end 288.75 144.3) (stroke (width 0.25) (type solid)) (layer "Edge.Cuts"))
 (gr_arc (start 354.25 147.25) (mid 354.03033 147.78033) (end 353.5 148) (stroke (width 0.25) (type solid)) (layer "Edge.Cuts"))
 (gr_line (start 354.25 147.25) (end 354.25 145.3) (stroke (width 0.25) (type solid)) (layer "Edge.Cuts"))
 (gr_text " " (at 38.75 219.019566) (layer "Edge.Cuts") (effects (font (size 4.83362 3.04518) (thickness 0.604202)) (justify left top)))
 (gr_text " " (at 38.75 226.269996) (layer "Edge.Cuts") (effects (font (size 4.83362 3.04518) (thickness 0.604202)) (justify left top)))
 (segment (start 222.66 153.5) (end 350.25 153.5) (width 0.4) (layer "F.Cu") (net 19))
 (segment (start 353.5 150.25) (end 350.25 153.5) (width 0.4) (layer "F.Cu") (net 19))
 (segment (start 221.66 152.5) (end 222.66 153.5) (width 0.4) (layer "F.Cu") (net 19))
 (segment (start 356.5 150.25) (end 353.5 150.25) (width 0.4) (layer "F.Cu") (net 19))
 (segment (start 220.62 151) (end 224.5 151) (width 0.4) (layer "F.Cu") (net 16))
 (segment (start 311.25 150.25) (end 331.77 150.25) (width 0.4) (layer "F.Cu") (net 16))
 (segment (start 219.12 152.5) (end 220.62 151) (width 0.4) (layer "F.Cu") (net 16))
 (segment (start 224.5 151) (end 226 152.5) (width 0.4) (layer "F.Cu") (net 16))
 (segment (start 309 152.5) (end 311.25 150.25) (width 0.4) (layer "F.Cu") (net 16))
 (segment (start 226 152.5) (end 309 152.5) (width 0.4) (layer "F.Cu") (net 16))
 (segment (start 240.85 150.25) (end 255.885 150.25) (width 0.4) (layer "F.Cu") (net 14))
 (segment (start 240.4 149.8) (end 240.85 150.25) (width 0.4) (layer "F.Cu") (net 14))
 (segment (start 216.74 149.8) (end 214.04 152.5) (width 0.4) (layer "F.Cu") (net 14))
 (segment (start 240.4 149.8) (end 216.74 149.8) (width 0.4) (layer "F.Cu") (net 14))
 (segment (start 200.04 151.2) (end 201.34 152.5) (width 0.4) (layer "F.Cu") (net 25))
 (segment (start 179.5 151.2) (end 200.04 151.2) (width 0.4) (layer "F.Cu") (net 25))
 (segment (start 197.95 153.35) (end 198.8 152.5) (width 0.4) (layer "F.Cu") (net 31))
 (segment (start 126 153.35) (end 197.95 153.35) (width 0.4) (layer "F.Cu") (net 31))
 (segment (start 123.15 150.5) (end 126 153.35) (width 0.4) (layer "F.Cu") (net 31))
 (segment (start 120.615 150.5) (end 123.15 150.5) (width 0.4) (layer "F.Cu") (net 31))
 (segment (start 51.27 158) (end 51.77 157.5) (width 0.4) (layer "F.Cu") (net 7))
 (segment (start 60.1 154.5) (end 57.1 157.5) (width 0.4) (layer "F.Cu") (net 7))
 (segment (start 60.1 154.5) (end 198.26 154.5) (width 0.4) (layer "F.Cu") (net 7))
 (segment (start 198.26 154.5) (end 198.8 155.04) (width 0.4) (layer "F.Cu") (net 7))
 (segment (start 57.1 157.5) (end 51.48 157.5) (width 0.4) (layer "F.Cu") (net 7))
 (segment (start 112 158) (end 114.5 155.5) (width 0.4) (layer "F.Cu") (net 23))
 (segment (start 197.5 157) (end 199 157) (width 0.4) (layer "F.Cu") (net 23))
 (segment (start 201.34 155.04) (end 199.38 157) (width 0.4) (layer "F.Cu") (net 23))
 (segment (start 199.38 157) (end 199 157) (width 0.4) (layer "F.Cu") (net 23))
 (segment (start 109.6 158) (end 112 158) (width 0.4) (layer "F.Cu") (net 23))
 (segment (start 196 155.5) (end 197.5 157) (width 0.4) (layer "F.Cu") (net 23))
 (segment (start 114.5 155.5) (end 196 155.5) (width 0.4) (layer "F.Cu") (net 23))
 (segment (start 203.88 155.04) (end 200.92 158) (width 0.4) (layer "F.Cu") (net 21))
 (segment (start 181.56 156.24) (end 180.3 157.5) (width 0.4) (layer "F.Cu") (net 21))
 (segment (start 200.92 158) (end 196.5 158) (width 0.4) (layer "F.Cu") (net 21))
 (segment (start 180.3 157.5) (end 167.23 157.5) (width 0.4) (layer "F.Cu") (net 21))
 (segment (start 194.74 156.24) (end 181.56 156.24) (width 0.4) (layer "F.Cu") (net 21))
 (segment (start 196.5 158) (end 194.74 156.24) (width 0.4) (layer "F.Cu") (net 21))
 (segment (start 238.2 159) (end 216 159) (width 0.4) (layer "F.Cu") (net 11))
 (segment (start 214.04 157.04) (end 214.04 155.04) (width 0.4) (layer "F.Cu") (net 11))
 (segment (start 216 159) (end 214.04 157.04) (width 0.4) (layer "F.Cu") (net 11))
 (segment (start 240.4 156.8) (end 238.2 159) (width 0.4) (layer "F.Cu") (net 11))
 (segment (start 293.25 157.75) (end 288.555 157.75) (width 0.4) (layer "F.Cu") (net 24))
 (segment (start 224 157.5) (end 222 157.5) (width 0.4) (layer "F.Cu") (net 24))
 (segment (start 219.12 155.04) (end 221.58 157.5) (width 0.4) (layer "F.Cu") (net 24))
 (segment (start 221.58 157.5) (end 222 157.5) (width 0.4) (layer "F.Cu") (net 24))
 (segment (start 288.555 157.75) (end 286.25 155.445) (width 0.4) (layer "F.Cu") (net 24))
 (segment (start 286.25 155.445) (end 226.055 155.445) (width 0.4) (layer "F.Cu") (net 24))
 (segment (start 226.055 155.445) (end 224 157.5) (width 0.4) (layer "F.Cu") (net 24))
 (segment (start 224.96 155.04) (end 225.5 154.5) (width 0.4) (layer "F.Cu") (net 8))
 (segment (start 361.6 154.5) (end 364.6 157.5) (width 0.4) (layer "F.Cu") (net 8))
 (segment (start 221.66 155.04) (end 224.96 155.04) (width 0.4) (layer "F.Cu") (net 8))
 (segment (start 364.6 157.5) (end 370.52 157.5) (width 0.4) (layer "F.Cu") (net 8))
 (segment (start 225.5 154.5) (end 361.6 154.5) (width 0.4) (layer "F.Cu") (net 8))
 (segment (start 218.08 151) (end 216.58 152.5) (width 0.2) (layer "B.Cu") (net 28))
 (segment (start 295 153) (end 234.5 153) (width 0.2) (layer "B.Cu") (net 28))
 (segment (start 232.5 151) (end 218.08 151) (width 0.2) (layer "B.Cu") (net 28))
 (segment (start 298.5 149.5) (end 295 153) (width 0.2) (layer "B.Cu") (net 28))
 (segment (start 234.5 153) (end 232.5 151) (width 0.2) (layer "B.Cu") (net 28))
 (segment (start 222.36 156.14) (end 217.68 156.14) (width 0.2) (layer "B.Cu") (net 29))
 (segment (start 217.68 156.14) (end 216.58 155.04) (width 0.2) (layer "B.Cu") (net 29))
 (segment (start 298.5 150.77) (end 295.92 153.35) (width 0.2) (layer "B.Cu") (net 29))
 (segment (start 225.15 153.35) (end 222.36 156.14) (width 0.2) (layer "B.Cu") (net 29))
 (segment (start 295.92 153.35) (end 225.15 153.35) (width 0.2) (layer "B.Cu") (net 29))
 (segment (start 204.92 151) (end 206.42 152.5) (width 0.2) (layer "B.Cu") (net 2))
 (segment (start 196 151) (end 204.92 151) (width 0.2) (layer "B.Cu") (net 2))
 (segment (start 79.5 149.73) (end 83.37 153.6) (width 0.2) (layer "B.Cu") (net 2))
 (segment (start 83.37 153.6) (end 193.4 153.6) (width 0.2) (layer "B.Cu") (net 2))
 (segment (start 193.4 153.6) (end 196 151) (width 0.2) (layer "B.Cu") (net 2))
 (segment (start 196.045 155.545) (end 197.5 157) (width 0.2) (layer "B.Cu") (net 3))
 (segment (start 79.5 151) (end 84.045 155.545) (width 0.2) (layer "B.Cu") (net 3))
 (segment (start 204.5 157) (end 204.5 156.96) (width 0.2) (layer "B.Cu") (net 3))
 (segment (start 197.5 157) (end 204.5 157) (width 0.2) (layer "B.Cu") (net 3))
 (segment (start 204.5 156.96) (end 206.42 155.04) (width 0.2) (layer "B.Cu") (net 3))
 (segment (start 84.045 155.545) (end 196.045 155.545) (width 0.2) (layer "B.Cu") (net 3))
 (segment (start 188 157.23) (end 188.12 157.35) (width 0.2) (layer "B.Cu") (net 26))
 (segment (start 205.665635 157.35) (end 207.86 155.155635) (width 0.2) (layer "B.Cu") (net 26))
 (segment (start 207.86 153.6) (end 208.96 152.5) (width 0.2) (layer "B.Cu") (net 26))
 (segment (start 207.86 155.155635) (end 207.86 153.6) (width 0.2) (layer "B.Cu") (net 26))
 (segment (start 188.12 157.35) (end 205.665635 157.35) (width 0.2) (layer "B.Cu") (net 26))
 (segment (start 188 158.5) (end 205.5 158.5) (width 0.2) (layer "B.Cu") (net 27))
 (segment (start 205.5 158.5) (end 208.96 155.04) (width 0.2) (layer "B.Cu") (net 27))
 (segment (start 226.51 156.49) (end 213.49 156.49) (width 0.2) (layer "B.Cu") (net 4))
 (segment (start 213.49 156.49) (end 212.6 155.6) (width 0.2) (layer "B.Cu") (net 4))
 (segment (start 347.77 155) (end 228 155) (width 0.2) (layer "B.Cu") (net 4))
 (segment (start 212.6 153.6) (end 211.5 152.5) (width 0.2) (layer "B.Cu") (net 4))
 (segment (start 350 157.23) (end 347.77 155) (width 0.2) (layer "B.Cu") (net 4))
 (segment (start 212.6 155.6) (end 212.6 153.6) (width 0.2) (layer "B.Cu") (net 4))
 (segment (start 228 155) (end 226.51 156.49) (width 0.2) (layer "B.Cu") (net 4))
 (segment (start 349 158.5) (end 346 155.5) (width 0.2) (layer "B.Cu") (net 5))
 (segment (start 228.5 155.5) (end 227.16 156.84) (width 0.2) (layer "B.Cu") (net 5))
 (segment (start 213.3 156.84) (end 211.5 155.04) (width 0.2) (layer "B.Cu") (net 5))
 (segment (start 346 155.5) (end 228.5 155.5) (width 0.2) (layer "B.Cu") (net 5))
 (segment (start 227.16 156.84) (end 213.3 156.84) (width 0.2) (layer "B.Cu") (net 5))
 (segment (start 350 158.5) (end 349 158.5) (width 0.2) (layer "B.Cu") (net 5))
 (segment (start 368.29 150.25) (end 361.73 150.25) (width 0.4) (layer "F.Cu") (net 18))
 (segment (start 369 149.54) (end 368.29 150.25) (width 0.4) (layer "F.Cu") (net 18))
 (segment (start 370 150) (end 369 151) (width 0.4) (layer "F.Cu") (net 18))
 (segment (start 369 149.54) (end 368.71 149.25) (width 0.4) (layer "F.Cu") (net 18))
 (segment (start 337 150.25) (end 346.5 150.25) (width 0.4) (layer "F.Cu") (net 15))
 (segment (start 346.5 150.25) (end 347.25 149.5) (width 0.4) (layer "F.Cu") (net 15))
 (segment (start 270.04 150.5) (end 271 149.54) (width 0.4) (layer "F.Cu") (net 13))
 (segment (start 261.115 150.5) (end 270.04 150.5) (width 0.4) (layer "F.Cu") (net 13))
 (segment (start 174.36 149.96) (end 174.4 150) (width 0.4) (layer "F.Cu") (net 12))
 (segment (start 167.5 149.96) (end 174.36 149.96) (width 0.4) (layer "F.Cu") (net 12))
 (segment (start 107 150.5) (end 106 149.5) (width 0.4) (layer "F.Cu") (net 17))
 (segment (start 115.385 150.5) (end 107 150.5) (width 0.4) (layer "F.Cu") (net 17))
 (segment (start 104.34 149.96) (end 104.5 149.8) (width 0.4) (layer "F.Cu") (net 17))
 (segment (start 46.25 157.5) (end 37.21 157.5) (width 0.4) (layer "F.Cu") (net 6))
 (segment (start 37.21 157.5) (end 36.25 158.46) (width 0.4) (layer "F.Cu") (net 6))
 (segment (start 104.27 157.5) (end 103.73 158.04) (width 0.4) (layer "F.Cu") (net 22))
 (segment (start 83.46 158.04) (end 83 158.5) (width 0.4) (layer "F.Cu") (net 22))
 (segment (start 103.73 158.04) (end 83.46 158.04) (width 0.4) (layer "F.Cu") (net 22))
 (segment (start 154 157.5) (end 153 158.5) (width 0.4) (layer "F.Cu") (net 20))
 (segment (start 162 157.5) (end 154 157.5) (width 0.4) (layer "F.Cu") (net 20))
 (segment (start 254.54 158.04) (end 255 158.5) (width 0.4) (layer "F.Cu") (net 10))
 (segment (start 245.5 158) (end 245.54 158.04) (width 0.4) (layer "F.Cu") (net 10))
 (segment (start 245.54 158.04) (end 254.54 158.04) (width 0.4) (layer "F.Cu") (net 10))
 (segment (start 307 158.5) (end 306.25 157.75) (width 0.4) (layer "F.Cu") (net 9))
 (segment (start 306.25 157.75) (end 298.48 157.75) (width 0.4) (layer "F.Cu") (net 9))
 (segment (start 375.75 157.5) (end 383.04 157.5) (width 0.4) (layer "F.Cu") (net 1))
 (segment (start 383.04 157.5) (end 384 158.46) (width 0.4) (layer "F.Cu") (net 1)))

